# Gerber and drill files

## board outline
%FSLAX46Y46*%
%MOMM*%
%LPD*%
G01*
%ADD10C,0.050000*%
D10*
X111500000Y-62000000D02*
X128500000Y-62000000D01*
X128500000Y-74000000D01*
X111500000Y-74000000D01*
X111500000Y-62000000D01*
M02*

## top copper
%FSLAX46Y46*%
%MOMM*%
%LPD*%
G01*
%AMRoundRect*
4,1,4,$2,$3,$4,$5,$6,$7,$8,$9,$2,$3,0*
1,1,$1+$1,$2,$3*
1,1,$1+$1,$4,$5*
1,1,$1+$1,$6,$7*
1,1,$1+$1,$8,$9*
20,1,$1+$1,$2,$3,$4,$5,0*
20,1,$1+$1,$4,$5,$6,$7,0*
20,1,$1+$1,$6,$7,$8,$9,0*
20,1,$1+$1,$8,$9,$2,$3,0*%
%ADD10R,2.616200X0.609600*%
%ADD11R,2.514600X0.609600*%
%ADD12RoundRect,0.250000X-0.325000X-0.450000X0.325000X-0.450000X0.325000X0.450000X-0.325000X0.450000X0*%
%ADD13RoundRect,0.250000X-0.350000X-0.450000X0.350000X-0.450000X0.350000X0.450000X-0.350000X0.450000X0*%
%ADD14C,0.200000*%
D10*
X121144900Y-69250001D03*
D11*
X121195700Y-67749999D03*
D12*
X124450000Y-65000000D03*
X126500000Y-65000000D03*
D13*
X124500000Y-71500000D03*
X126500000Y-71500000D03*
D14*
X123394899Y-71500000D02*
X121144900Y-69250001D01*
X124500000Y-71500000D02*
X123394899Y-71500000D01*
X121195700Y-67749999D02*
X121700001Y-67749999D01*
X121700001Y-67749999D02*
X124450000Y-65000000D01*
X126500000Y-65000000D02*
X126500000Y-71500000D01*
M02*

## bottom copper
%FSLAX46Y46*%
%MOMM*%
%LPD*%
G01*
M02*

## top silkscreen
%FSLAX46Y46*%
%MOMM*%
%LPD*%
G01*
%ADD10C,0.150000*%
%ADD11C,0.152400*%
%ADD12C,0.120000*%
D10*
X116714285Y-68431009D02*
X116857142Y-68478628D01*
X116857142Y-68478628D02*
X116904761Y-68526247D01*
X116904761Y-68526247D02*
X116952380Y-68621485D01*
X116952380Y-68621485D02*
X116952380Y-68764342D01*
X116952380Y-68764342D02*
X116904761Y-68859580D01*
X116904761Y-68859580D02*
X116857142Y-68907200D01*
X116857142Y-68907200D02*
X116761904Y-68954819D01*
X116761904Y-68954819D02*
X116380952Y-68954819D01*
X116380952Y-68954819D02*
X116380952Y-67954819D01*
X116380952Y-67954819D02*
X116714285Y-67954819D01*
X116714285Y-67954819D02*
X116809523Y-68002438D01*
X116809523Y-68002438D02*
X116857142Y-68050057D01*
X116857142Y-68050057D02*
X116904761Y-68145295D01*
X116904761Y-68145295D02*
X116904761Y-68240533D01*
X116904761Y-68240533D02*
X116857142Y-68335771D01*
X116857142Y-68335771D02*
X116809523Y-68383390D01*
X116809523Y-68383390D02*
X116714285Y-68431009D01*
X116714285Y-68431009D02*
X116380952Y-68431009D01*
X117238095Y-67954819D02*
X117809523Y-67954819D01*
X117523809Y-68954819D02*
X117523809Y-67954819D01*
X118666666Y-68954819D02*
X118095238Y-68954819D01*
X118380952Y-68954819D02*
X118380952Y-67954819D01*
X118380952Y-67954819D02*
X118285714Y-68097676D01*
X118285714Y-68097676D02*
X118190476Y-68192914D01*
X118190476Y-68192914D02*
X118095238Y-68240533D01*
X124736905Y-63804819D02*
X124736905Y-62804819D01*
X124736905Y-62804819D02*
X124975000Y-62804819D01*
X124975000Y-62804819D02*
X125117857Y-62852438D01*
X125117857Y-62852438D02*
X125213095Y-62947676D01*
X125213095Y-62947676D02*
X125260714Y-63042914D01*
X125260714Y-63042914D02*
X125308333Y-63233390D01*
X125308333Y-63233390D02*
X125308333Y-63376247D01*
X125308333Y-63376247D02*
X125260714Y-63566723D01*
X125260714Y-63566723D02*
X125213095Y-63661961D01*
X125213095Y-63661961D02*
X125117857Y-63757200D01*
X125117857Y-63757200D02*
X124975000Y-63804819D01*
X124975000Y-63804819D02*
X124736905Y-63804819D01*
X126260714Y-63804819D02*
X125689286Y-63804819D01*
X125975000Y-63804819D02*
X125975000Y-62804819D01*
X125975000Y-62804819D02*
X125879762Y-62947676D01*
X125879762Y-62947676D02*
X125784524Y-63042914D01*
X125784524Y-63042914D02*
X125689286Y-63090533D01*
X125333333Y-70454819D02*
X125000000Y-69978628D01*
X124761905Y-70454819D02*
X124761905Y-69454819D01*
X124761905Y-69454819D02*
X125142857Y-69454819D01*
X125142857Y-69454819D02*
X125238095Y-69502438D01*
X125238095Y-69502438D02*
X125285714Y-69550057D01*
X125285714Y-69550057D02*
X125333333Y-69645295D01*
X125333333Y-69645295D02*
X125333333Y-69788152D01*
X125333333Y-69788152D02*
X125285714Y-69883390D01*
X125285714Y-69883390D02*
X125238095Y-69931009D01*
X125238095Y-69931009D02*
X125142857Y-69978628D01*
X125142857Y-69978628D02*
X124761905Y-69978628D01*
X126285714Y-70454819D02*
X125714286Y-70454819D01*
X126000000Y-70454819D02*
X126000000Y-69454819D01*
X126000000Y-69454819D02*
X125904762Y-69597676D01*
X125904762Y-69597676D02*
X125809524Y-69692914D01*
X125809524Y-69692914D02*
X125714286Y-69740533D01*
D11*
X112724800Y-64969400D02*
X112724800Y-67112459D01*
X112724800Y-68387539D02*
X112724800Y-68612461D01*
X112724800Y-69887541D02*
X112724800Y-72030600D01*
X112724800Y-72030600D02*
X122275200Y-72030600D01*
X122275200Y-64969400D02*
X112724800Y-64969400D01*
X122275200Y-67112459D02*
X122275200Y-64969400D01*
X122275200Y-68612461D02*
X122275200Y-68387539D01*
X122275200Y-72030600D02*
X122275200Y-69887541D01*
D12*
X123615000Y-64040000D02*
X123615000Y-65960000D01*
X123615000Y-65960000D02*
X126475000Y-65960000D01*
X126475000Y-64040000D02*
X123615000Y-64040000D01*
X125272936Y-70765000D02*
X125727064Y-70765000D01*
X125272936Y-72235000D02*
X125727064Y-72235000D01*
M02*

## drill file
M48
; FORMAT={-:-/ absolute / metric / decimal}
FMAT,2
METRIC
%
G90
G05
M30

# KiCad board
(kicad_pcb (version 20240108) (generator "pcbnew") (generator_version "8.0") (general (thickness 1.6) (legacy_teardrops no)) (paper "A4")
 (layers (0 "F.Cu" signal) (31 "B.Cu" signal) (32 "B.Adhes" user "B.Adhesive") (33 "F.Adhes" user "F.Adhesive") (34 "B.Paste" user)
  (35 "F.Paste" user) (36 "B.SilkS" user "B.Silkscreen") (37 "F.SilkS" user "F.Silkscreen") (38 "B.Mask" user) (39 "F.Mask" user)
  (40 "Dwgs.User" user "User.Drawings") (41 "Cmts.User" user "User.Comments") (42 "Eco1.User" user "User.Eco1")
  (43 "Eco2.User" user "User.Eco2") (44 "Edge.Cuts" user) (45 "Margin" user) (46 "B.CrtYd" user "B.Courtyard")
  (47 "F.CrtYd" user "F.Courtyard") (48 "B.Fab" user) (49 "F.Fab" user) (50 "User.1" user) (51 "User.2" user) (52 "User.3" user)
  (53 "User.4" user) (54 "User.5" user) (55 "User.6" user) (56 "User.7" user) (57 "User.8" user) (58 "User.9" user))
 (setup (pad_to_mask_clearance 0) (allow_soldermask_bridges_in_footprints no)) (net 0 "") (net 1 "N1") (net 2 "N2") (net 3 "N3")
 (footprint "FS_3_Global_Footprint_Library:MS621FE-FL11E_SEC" (layer "F.Cu") (at 117.5 68.5 180)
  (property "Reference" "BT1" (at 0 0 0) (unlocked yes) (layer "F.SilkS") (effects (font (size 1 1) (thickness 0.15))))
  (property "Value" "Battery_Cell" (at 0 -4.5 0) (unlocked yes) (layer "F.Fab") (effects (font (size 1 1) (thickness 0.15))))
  (fp_line (start 4.7752 3.5306) (end 4.7752 1.387541) (stroke (width 0.1524) (type solid)) (layer "F.SilkS"))
  (fp_line (start 4.7752 0.112461) (end 4.7752 -0.112461) (stroke (width 0.1524) (type solid)) (layer "F.SilkS"))
  (fp_line (start 4.7752 -1.387541) (end 4.7752 -3.5306) (stroke (width 0.1524) (type solid)) (layer "F.SilkS"))
  (fp_line (start 4.7752 -3.5306) (end -4.7752 -3.5306) (stroke (width 0.1524) (type solid)) (layer "F.SilkS"))
  (fp_line (start -4.7752 3.5306) (end 4.7752 3.5306) (stroke (width 0.1524) (type solid)) (layer "F.SilkS"))
  (fp_line (start -4.7752 1.387541) (end -4.7752 3.5306) (stroke (width 0.1524) (type solid)) (layer "F.SilkS"))
  (fp_line (start -4.7752 -0.112461) (end -4.7752 0.112461) (stroke (width 0.1524) (type solid)) (layer "F.SilkS"))
  (fp_line (start -4.7752 -3.5306) (end -4.7752 -1.387541) (stroke (width 0.1524) (type solid)) (layer "F.SilkS"))
  (pad "1" smd rect (at -3.6449 -0.750001 180) (size 2.6162 0.6096) (layers "F.Cu" "F.Paste" "F.Mask") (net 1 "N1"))
  (pad "2" smd rect (at -3.6957 0.750001 180) (size 2.5146 0.6096) (layers "F.Cu" "F.Paste" "F.Mask") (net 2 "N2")))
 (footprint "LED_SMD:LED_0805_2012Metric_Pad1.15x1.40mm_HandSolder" (layer "F.Cu") (at 125.475 65)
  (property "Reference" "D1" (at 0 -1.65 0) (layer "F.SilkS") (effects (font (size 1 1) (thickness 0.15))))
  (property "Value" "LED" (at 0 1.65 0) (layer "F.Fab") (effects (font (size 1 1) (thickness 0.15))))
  (fp_line (start -1.86 -0.96) (end -1.86 0.96) (stroke (width 0.12) (type solid)) (layer "F.SilkS"))
  (fp_line (start -1.86 0.96) (end 1 0.96) (stroke (width 0.12) (type solid)) (layer "F.SilkS"))
  (fp_line (start 1 -0.96) (end -1.86 -0.96) (stroke (width 0.12) (type solid)) (layer "F.SilkS"))
  (pad "1" smd roundrect (at -1.025 0) (size 1.15 1.4) (layers "F.Cu" "F.Paste" "F.Mask") (roundrect_rratio 0.217391) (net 2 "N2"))
  (pad "2" smd roundrect (at 1.025 0) (size 1.15 1.4) (layers "F.Cu" "F.Paste" "F.Mask") (roundrect_rratio 0.217391) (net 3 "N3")))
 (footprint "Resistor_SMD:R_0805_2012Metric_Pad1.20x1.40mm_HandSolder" (layer "F.Cu") (at 125.5 71.5)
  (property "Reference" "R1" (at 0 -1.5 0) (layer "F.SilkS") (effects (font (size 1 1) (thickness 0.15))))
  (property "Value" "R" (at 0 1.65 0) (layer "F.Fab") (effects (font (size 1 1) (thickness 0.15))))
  (fp_line (start -0.227064 -0.735) (end 0.227064 -0.735) (stroke (width 0.12) (type solid)) (layer "F.SilkS"))
  (fp_line (start -0.227064 0.735) (end 0.227064 0.735) (stroke (width 0.12) (type solid)) (layer "F.SilkS"))
  (pad "1" smd roundrect (at -1 0) (size 1.2 1.4) (layers "F.Cu" "F.Paste" "F.Mask") (roundrect_rratio 0.208333) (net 1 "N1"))
  (pad "2" smd roundrect (at 1 0) (size 1.2 1.4) (layers "F.Cu" "F.Paste" "F.Mask") (roundrect_rratio 0.208333) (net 3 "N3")))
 (gr_rect (start 111.5 62) (end 128.5 74) (stroke (width 0.05) (type default)) (fill none) (layer "Edge.Cuts"))
 (segment (start 123.394899 71.5) (end 121.1449 69.250001) (width 0.2) (layer "F.Cu") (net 1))
 (segment (start 124.5 71.5) (end 123.394899 71.5) (width 0.2) (layer "F.Cu") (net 1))
 (segment (start 121.1957 67.749999) (end 121.700001 67.749999) (width 0.2) (layer "F.Cu") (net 2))
 (segment (start 121.700001 67.749999) (end 124.45 65) (width 0.2) (layer "F.Cu") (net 2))
 (segment (start 126.5 65) (end 126.5 71.5) (width 0.2) (layer "F.Cu") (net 3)))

